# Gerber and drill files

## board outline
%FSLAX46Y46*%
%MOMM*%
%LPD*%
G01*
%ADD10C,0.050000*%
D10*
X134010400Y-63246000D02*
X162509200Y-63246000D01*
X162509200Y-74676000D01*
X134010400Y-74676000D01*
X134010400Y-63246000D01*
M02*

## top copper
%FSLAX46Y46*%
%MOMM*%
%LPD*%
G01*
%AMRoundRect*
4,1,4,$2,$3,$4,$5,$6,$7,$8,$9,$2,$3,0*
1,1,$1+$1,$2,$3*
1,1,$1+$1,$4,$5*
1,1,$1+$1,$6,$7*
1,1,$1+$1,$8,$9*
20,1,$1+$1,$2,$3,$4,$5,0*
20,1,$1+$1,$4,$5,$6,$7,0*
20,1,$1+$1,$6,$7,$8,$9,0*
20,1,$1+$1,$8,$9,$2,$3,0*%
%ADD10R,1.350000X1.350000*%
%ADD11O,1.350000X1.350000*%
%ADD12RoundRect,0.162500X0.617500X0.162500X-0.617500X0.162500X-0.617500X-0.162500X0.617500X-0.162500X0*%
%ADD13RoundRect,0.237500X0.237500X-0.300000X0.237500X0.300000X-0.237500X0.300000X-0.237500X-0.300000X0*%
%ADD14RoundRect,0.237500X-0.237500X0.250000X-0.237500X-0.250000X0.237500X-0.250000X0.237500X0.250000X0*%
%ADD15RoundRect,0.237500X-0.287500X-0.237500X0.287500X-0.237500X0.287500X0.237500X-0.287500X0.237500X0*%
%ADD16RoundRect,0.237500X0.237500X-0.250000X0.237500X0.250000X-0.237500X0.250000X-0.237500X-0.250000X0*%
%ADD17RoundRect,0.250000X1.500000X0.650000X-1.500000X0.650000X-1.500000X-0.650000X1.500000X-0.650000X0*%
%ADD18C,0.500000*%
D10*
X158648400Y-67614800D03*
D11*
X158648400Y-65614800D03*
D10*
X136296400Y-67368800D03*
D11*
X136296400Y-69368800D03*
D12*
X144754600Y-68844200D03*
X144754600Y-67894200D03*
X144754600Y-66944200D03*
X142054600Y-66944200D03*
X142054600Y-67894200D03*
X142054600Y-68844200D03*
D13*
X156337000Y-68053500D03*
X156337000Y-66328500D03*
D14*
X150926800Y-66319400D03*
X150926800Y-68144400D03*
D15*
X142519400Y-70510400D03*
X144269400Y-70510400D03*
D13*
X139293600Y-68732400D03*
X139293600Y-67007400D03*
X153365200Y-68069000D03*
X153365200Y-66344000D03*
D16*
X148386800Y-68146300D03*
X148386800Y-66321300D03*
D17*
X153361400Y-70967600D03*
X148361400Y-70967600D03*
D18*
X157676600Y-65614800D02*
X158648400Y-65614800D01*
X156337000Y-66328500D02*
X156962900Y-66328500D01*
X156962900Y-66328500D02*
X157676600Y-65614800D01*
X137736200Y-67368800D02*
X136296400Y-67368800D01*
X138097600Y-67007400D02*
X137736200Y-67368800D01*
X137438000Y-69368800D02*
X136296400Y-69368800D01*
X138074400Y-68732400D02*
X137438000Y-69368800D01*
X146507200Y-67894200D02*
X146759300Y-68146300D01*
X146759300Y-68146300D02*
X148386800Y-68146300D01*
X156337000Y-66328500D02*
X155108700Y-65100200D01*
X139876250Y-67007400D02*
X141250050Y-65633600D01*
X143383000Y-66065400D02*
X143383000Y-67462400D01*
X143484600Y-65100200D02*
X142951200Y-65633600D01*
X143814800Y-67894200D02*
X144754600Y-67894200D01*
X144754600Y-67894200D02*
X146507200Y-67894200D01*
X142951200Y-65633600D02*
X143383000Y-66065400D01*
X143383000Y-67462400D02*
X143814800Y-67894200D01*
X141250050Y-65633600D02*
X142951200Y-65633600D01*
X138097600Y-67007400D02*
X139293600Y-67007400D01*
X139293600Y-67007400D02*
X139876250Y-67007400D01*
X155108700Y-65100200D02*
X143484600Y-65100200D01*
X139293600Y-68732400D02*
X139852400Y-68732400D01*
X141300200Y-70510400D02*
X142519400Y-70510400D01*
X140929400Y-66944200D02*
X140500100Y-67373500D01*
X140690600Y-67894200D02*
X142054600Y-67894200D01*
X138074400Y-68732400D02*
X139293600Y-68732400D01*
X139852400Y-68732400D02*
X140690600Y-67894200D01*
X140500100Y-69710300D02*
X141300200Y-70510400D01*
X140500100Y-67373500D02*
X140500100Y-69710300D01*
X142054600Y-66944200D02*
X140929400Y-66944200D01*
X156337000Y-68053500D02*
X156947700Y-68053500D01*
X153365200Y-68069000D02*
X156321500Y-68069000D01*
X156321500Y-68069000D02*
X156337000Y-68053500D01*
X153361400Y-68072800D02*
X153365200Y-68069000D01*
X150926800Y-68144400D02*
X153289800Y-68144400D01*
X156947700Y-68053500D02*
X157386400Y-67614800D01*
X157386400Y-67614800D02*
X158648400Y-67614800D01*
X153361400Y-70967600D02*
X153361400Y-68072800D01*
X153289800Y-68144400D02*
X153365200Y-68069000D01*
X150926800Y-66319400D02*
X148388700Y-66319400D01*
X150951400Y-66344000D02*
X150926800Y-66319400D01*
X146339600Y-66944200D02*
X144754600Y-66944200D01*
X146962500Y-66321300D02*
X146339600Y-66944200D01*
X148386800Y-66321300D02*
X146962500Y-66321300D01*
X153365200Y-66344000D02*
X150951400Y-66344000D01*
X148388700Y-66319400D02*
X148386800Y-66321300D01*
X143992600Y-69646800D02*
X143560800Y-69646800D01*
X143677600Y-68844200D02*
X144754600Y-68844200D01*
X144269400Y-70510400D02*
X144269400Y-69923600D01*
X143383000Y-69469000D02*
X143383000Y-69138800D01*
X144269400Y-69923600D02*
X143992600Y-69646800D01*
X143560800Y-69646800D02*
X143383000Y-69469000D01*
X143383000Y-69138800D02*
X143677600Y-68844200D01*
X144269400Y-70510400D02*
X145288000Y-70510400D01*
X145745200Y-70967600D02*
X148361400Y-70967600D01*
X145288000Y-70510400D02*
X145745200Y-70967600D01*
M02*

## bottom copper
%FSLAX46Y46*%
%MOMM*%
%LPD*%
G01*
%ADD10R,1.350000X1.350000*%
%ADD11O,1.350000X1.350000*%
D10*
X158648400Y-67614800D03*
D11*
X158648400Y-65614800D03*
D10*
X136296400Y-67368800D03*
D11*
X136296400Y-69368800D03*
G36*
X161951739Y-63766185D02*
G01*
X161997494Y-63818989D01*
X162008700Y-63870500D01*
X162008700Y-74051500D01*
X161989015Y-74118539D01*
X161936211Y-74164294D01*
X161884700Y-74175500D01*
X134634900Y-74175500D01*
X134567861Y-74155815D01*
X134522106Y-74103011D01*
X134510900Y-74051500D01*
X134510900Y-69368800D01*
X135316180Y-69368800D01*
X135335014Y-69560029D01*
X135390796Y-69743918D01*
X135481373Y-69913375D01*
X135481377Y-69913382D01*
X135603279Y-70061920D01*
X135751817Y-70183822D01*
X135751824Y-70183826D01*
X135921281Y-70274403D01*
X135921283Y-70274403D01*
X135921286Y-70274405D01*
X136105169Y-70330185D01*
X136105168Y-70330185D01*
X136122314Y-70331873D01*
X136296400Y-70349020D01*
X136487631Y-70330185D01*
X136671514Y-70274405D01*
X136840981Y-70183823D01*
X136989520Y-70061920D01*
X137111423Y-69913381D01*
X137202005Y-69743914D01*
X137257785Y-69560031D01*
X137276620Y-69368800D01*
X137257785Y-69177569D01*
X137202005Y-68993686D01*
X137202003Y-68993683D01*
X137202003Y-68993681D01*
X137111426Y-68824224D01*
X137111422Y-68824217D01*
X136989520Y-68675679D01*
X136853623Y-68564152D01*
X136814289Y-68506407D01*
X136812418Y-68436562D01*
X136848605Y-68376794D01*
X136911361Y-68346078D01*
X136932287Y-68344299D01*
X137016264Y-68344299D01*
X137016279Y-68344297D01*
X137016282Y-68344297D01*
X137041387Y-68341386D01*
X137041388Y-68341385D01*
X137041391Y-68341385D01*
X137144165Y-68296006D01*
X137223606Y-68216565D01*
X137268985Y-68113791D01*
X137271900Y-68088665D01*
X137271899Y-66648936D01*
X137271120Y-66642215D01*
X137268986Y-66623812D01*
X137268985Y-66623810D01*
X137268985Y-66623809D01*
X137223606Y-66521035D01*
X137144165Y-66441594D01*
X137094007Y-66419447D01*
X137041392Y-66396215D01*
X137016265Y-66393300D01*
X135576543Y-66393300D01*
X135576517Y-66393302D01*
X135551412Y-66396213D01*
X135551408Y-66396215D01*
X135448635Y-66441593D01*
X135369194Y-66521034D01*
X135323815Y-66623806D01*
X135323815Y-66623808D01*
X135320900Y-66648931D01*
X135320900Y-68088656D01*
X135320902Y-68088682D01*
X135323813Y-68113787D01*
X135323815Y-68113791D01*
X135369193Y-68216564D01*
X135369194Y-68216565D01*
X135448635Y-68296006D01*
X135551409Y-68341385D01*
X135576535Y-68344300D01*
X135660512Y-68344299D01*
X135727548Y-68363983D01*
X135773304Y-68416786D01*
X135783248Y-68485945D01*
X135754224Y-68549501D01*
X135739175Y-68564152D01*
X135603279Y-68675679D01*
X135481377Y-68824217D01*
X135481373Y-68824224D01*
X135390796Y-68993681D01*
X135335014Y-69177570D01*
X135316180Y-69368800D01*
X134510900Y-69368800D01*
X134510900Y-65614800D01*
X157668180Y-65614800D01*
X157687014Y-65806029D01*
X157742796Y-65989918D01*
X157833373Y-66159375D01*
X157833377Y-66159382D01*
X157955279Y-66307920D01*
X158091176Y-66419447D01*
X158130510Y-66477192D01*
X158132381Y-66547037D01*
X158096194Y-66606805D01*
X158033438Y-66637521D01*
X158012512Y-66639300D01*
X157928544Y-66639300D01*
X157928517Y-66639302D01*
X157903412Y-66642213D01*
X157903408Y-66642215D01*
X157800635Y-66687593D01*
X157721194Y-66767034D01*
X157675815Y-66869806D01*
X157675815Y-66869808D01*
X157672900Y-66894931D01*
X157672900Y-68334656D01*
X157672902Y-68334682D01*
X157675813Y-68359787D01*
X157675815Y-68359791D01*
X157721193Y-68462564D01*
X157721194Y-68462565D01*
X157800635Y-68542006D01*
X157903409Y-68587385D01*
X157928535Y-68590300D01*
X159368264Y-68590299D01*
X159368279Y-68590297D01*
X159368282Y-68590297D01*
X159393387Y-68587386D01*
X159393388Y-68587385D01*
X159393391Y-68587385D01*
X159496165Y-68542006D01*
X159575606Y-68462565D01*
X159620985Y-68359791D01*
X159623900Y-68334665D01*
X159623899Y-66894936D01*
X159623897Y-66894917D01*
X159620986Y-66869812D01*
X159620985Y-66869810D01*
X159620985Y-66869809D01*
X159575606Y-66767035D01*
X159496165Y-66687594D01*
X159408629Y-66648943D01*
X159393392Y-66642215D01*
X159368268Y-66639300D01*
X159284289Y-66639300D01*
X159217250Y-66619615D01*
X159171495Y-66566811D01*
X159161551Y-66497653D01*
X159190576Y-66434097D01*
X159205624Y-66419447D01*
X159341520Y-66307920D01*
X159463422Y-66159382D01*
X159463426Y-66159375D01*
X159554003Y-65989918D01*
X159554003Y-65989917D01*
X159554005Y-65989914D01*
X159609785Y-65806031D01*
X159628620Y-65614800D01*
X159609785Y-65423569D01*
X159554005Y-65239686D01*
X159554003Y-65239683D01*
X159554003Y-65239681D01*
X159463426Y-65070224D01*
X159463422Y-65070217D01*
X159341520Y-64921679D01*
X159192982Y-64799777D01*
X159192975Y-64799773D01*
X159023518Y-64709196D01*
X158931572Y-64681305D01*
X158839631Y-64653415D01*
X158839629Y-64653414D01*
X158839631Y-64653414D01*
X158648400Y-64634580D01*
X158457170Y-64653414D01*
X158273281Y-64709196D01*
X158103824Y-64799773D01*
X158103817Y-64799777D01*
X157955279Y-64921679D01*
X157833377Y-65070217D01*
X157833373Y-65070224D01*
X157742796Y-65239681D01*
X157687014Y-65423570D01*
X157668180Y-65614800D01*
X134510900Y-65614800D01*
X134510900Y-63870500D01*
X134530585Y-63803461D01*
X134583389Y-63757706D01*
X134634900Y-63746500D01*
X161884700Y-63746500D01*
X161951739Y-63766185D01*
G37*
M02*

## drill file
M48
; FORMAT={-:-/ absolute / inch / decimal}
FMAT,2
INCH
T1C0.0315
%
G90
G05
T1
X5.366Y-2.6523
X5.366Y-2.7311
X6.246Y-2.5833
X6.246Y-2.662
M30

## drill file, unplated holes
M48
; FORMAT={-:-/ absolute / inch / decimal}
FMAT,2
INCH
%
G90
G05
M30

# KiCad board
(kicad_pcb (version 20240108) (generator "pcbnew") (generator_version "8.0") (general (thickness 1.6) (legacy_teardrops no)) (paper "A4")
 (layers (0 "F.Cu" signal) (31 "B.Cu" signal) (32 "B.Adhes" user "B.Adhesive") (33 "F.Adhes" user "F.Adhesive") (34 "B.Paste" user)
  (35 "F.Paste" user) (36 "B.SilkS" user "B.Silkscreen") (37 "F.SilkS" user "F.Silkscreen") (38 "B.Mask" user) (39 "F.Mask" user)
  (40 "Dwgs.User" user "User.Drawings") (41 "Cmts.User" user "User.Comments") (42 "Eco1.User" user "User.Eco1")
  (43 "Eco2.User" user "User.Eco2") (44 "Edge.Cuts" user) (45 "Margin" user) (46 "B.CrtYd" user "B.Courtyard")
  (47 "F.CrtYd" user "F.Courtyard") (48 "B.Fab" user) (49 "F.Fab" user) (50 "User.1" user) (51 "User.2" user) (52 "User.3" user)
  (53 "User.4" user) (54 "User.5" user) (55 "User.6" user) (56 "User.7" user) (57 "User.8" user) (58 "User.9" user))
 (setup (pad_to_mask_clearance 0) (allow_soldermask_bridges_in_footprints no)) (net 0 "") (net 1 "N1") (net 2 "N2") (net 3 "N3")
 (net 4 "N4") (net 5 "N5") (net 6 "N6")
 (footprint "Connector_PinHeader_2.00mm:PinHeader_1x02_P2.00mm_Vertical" (layer "F.Cu") (at 136.2964 67.3688)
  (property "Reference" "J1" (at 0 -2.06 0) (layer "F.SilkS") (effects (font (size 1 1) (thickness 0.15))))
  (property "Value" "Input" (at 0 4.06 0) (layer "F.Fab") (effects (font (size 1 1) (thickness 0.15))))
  (pad "1" thru_hole rect (at 0 0) (size 1.35 1.35) (drill 0.8) (layers "*.Cu" "*.Mask") (remove_unused_layers no) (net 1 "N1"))
  (pad "2" thru_hole oval (at 0 2) (size 1.35 1.35) (drill 0.8) (layers "*.Cu" "*.Mask") (remove_unused_layers no) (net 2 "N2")))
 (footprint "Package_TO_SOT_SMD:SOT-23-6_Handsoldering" (layer "F.Cu") (at 143.4046 67.8942 180)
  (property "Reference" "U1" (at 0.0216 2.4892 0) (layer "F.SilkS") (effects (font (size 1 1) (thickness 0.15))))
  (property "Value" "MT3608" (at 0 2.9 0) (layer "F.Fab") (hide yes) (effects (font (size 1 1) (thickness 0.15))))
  (pad "1" smd roundrect (at -1.35 -0.95 180) (size 1.56 0.65) (layers "F.Cu" "F.Paste" "F.Mask") (roundrect_rratio 0.25) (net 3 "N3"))
  (pad "2" smd roundrect (at -1.35 0 180) (size 1.56 0.65) (layers "F.Cu" "F.Paste" "F.Mask") (roundrect_rratio 0.25) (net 1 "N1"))
  (pad "3" smd roundrect (at -1.35 0.95 180) (size 1.56 0.65) (layers "F.Cu" "F.Paste" "F.Mask") (roundrect_rratio 0.25) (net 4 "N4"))
  (pad "4" smd roundrect (at 1.35 0.95 180) (size 1.56 0.65) (layers "F.Cu" "F.Paste" "F.Mask") (roundrect_rratio 0.25) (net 2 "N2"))
  (pad "5" smd roundrect (at 1.35 0 180) (size 1.56 0.65) (layers "F.Cu" "F.Paste" "F.Mask") (roundrect_rratio 0.25) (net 2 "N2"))
  (pad "6" smd roundrect (at 1.35 -0.95 180) (size 1.56 0.65) (layers "F.Cu" "F.Paste" "F.Mask") (roundrect_rratio 0.25) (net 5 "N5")))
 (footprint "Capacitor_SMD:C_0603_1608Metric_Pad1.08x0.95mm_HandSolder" (layer "F.Cu") (at 156.337 67.191 90)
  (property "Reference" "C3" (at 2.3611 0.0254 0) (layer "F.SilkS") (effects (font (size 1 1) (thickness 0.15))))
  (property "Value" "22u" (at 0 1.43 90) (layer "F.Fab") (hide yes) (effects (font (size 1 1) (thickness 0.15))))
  (pad "1" smd roundrect (at -0.8625 0 90) (size 1.075 0.95) (layers "F.Cu" "F.Paste" "F.Mask") (roundrect_rratio 0.25) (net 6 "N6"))
  (pad "2" smd roundrect (at 0.8625 0 90) (size 1.075 0.95) (layers "F.Cu" "F.Paste" "F.Mask") (roundrect_rratio 0.25) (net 1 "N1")))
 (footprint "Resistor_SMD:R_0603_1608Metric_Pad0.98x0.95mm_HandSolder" (layer "F.Cu") (at 150.9268 67.2319 -90)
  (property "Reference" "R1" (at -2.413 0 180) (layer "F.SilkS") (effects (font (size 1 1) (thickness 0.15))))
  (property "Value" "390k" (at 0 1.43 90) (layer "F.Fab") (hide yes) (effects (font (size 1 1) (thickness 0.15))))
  (pad "1" smd roundrect (at -0.9125 0 270) (size 0.975 0.95) (layers "F.Cu" "F.Paste" "F.Mask") (roundrect_rratio 0.25) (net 4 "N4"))
  (pad "2" smd roundrect (at 0.9125 0 270) (size 0.975 0.95) (layers "F.Cu" "F.Paste" "F.Mask") (roundrect_rratio 0.25) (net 6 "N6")))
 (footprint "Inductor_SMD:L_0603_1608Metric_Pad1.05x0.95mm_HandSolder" (layer "F.Cu") (at 143.3944 70.5104)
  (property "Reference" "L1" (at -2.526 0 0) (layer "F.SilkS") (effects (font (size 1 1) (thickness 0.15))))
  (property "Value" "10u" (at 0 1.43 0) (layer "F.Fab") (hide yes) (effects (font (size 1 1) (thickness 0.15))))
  (pad "1" smd roundrect (at -0.875 0) (size 1.05 0.95) (layers "F.Cu" "F.Paste" "F.Mask") (roundrect_rratio 0.25) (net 2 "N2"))
  (pad "2" smd roundrect (at 0.875 0) (size 1.05 0.95) (layers "F.Cu" "F.Paste" "F.Mask") (roundrect_rratio 0.25) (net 3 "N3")))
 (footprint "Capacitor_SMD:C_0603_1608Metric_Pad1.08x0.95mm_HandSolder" (layer "F.Cu") (at 139.2936 67.8699 90)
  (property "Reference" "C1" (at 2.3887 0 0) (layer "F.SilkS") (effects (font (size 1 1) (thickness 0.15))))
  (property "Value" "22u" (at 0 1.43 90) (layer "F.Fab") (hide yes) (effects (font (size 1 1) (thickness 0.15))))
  (pad "1" smd roundrect (at -0.8625 0 90) (size 1.075 0.95) (layers "F.Cu" "F.Paste" "F.Mask") (roundrect_rratio 0.25) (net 2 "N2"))
  (pad "2" smd roundrect (at 0.8625 0 90) (size 1.075 0.95) (layers "F.Cu" "F.Paste" "F.Mask") (roundrect_rratio 0.25) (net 1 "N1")))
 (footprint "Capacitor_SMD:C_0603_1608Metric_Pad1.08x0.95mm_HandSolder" (layer "F.Cu") (at 153.3652 67.2065 90)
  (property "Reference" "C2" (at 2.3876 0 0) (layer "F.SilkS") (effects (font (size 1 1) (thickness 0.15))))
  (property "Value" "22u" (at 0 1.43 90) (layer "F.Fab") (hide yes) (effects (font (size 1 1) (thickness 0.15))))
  (pad "1" smd roundrect (at -0.8625 0 90) (size 1.075 0.95) (layers "F.Cu" "F.Paste" "F.Mask") (roundrect_rratio 0.25) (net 6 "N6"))
  (pad "2" smd roundrect (at 0.8625 0 90) (size 1.075 0.95) (layers "F.Cu" "F.Paste" "F.Mask") (roundrect_rratio 0.25) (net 4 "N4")))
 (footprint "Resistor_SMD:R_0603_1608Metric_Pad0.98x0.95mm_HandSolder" (layer "F.Cu") (at 148.3868 67.2338 90)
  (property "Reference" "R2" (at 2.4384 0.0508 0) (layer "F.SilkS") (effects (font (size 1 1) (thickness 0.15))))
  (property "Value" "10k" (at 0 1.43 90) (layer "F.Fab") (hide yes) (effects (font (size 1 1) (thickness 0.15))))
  (pad "1" smd roundrect (at -0.9125 0 90) (size 0.975 0.95) (layers "F.Cu" "F.Paste" "F.Mask") (roundrect_rratio 0.25) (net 1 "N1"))
  (pad "2" smd roundrect (at 0.9125 0 90) (size 0.975 0.95) (layers "F.Cu" "F.Paste" "F.Mask") (roundrect_rratio 0.25) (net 4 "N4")))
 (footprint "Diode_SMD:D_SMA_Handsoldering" (layer "F.Cu") (at 150.8614 70.9676 180)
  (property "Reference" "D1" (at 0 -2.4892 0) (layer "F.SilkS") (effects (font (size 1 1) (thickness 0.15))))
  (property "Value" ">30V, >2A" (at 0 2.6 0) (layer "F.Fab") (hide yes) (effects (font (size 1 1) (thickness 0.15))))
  (pad "1" smd roundrect (at -2.5 0 180) (size 3.5 1.8) (layers "F.Cu" "F.Paste" "F.Mask") (roundrect_rratio 0.1388888889) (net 6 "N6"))
  (pad "2" smd roundrect (at 2.5 0 180) (size 3.5 1.8) (layers "F.Cu" "F.Paste" "F.Mask") (roundrect_rratio 0.1388888889) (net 3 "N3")))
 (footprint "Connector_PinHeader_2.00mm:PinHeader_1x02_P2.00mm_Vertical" (layer "F.Cu") (at 158.6484 67.6148 180)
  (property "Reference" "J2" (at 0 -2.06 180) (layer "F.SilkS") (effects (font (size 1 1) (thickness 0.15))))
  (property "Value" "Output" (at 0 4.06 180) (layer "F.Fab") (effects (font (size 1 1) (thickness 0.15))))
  (pad "1" thru_hole rect (at 0 0 180) (size 1.35 1.35) (drill 0.8) (layers "*.Cu" "*.Mask") (remove_unused_layers no) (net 6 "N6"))
  (pad "2" thru_hole oval (at 0 2 180) (size 1.35 1.35) (drill 0.8) (layers "*.Cu" "*.Mask") (remove_unused_layers no) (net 1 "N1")))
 (gr_rect (start 134.0104 63.246) (end 162.5092 74.676) (stroke (width 0.05) (type default)) (fill none) (layer "Edge.Cuts"))
 (segment (start 146.5072 67.8942) (end 146.7593 68.1463) (width 0.5) (layer "F.Cu") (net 1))
 (segment (start 146.7593 68.1463) (end 148.3868 68.1463) (width 0.5) (layer "F.Cu") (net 1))
 (segment (start 156.337 66.3285) (end 155.1087 65.1002) (width 0.5) (layer "F.Cu") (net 1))
 (segment (start 138.0976 67.0074) (end 137.7362 67.3688) (width 0.5) (layer "F.Cu") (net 1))
 (segment (start 139.87625 67.0074) (end 141.25005 65.6336) (width 0.5) (layer "F.Cu") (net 1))
 (segment (start 143.383 66.0654) (end 143.383 67.4624) (width 0.5) (layer "F.Cu") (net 1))
 (segment (start 143.4846 65.1002) (end 142.9512 65.6336) (width 0.5) (layer "F.Cu") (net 1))
 (segment (start 156.9629 66.3285) (end 157.6766 65.6148) (width 0.5) (layer "F.Cu") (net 1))
 (segment (start 143.8148 67.8942) (end 144.7546 67.8942) (width 0.5) (layer "F.Cu") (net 1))
 (segment (start 144.7546 67.8942) (end 146.5072 67.8942) (width 0.5) (layer "F.Cu") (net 1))
 (segment (start 156.337 66.3285) (end 156.9629 66.3285) (width 0.5) (layer "F.Cu") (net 1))
 (segment (start 142.9512 65.6336) (end 143.383 66.0654) (width 0.5) (layer "F.Cu") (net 1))
 (segment (start 143.383 67.4624) (end 143.8148 67.8942) (width 0.5) (layer "F.Cu") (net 1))
 (segment (start 141.25005 65.6336) (end 142.9512 65.6336) (width 0.5) (layer "F.Cu") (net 1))
 (segment (start 138.0976 67.0074) (end 139.2936 67.0074) (width 0.5) (layer "F.Cu") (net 1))
 (segment (start 137.7362 67.3688) (end 136.2964 67.3688) (width 0.5) (layer "F.Cu") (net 1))
 (segment (start 157.6766 65.6148) (end 158.6484 65.6148) (width 0.5) (layer "F.Cu") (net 1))
 (segment (start 139.2936 67.0074) (end 139.87625 67.0074) (width 0.5) (layer "F.Cu") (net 1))
 (segment (start 155.1087 65.1002) (end 143.4846 65.1002) (width 0.5) (layer "F.Cu") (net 1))
 (segment (start 137.438 69.3688) (end 136.2964 69.3688) (width 0.5) (layer "F.Cu") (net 2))
 (segment (start 139.2936 68.7324) (end 139.8524 68.7324) (width 0.5) (layer "F.Cu") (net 2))
 (segment (start 141.3002 70.5104) (end 142.5194 70.5104) (width 0.5) (layer "F.Cu") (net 2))
 (segment (start 140.9294 66.9442) (end 140.5001 67.3735) (width 0.5) (layer "F.Cu") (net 2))
 (segment (start 140.6906 67.8942) (end 142.0546 67.8942) (width 0.5) (layer "F.Cu") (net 2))
 (segment (start 138.0744 68.7324) (end 139.2936 68.7324) (width 0.5) (layer "F.Cu") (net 2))
 (segment (start 139.8524 68.7324) (end 140.6906 67.8942) (width 0.5) (layer "F.Cu") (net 2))
 (segment (start 140.5001 69.7103) (end 141.3002 70.5104) (width 0.5) (layer "F.Cu") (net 2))
 (segment (start 138.0744 68.7324) (end 137.438 69.3688) (width 0.5) (layer "F.Cu") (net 2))
 (segment (start 140.5001 67.3735) (end 140.5001 69.7103) (width 0.5) (layer "F.Cu") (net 2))
 (segment (start 142.0546 66.9442) (end 140.9294 66.9442) (width 0.5) (layer "F.Cu") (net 2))
 (segment (start 156.337 68.0535) (end 156.9477 68.0535) (width 0.5) (layer "F.Cu") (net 6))
 (segment (start 153.3652 68.069) (end 156.3215 68.069) (width 0.5) (layer "F.Cu") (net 6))
 (segment (start 156.3215 68.069) (end 156.337 68.0535) (width 0.5) (layer "F.Cu") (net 6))
 (segment (start 153.3614 68.0728) (end 153.3652 68.069) (width 0.5) (layer "F.Cu") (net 6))
 (segment (start 150.9268 68.1444) (end 153.2898 68.1444) (width 0.5) (layer "F.Cu") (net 6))
 (segment (start 156.9477 68.0535) (end 157.3864 67.6148) (width 0.5) (layer "F.Cu") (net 6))
 (segment (start 157.3864 67.6148) (end 158.6484 67.6148) (width 0.5) (layer "F.Cu") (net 6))
 (segment (start 153.3614 70.9676) (end 153.3614 68.0728) (width 0.5) (layer "F.Cu") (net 6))
 (segment (start 153.2898 68.1444) (end 153.3652 68.069) (width 0.5) (layer "F.Cu") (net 6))
 (segment (start 150.9268 66.3194) (end 148.3887 66.3194) (width 0.5) (layer "F.Cu") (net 4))
 (segment (start 150.9514 66.344) (end 150.9268 66.3194) (width 0.5) (layer "F.Cu") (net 4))
 (segment (start 146.3396 66.9442) (end 144.7546 66.9442) (width 0.5) (layer "F.Cu") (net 4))
 (segment (start 146.9625 66.3213) (end 146.3396 66.9442) (width 0.5) (layer "F.Cu") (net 4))
 (segment (start 148.3868 66.3213) (end 146.9625 66.3213) (width 0.5) (layer "F.Cu") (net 4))
 (segment (start 153.3652 66.344) (end 150.9514 66.344) (width 0.5) (layer "F.Cu") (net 4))
 (segment (start 148.3887 66.3194) (end 148.3868 66.3213) (width 0.5) (layer "F.Cu") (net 4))
 (segment (start 143.9926 69.6468) (end 143.5608 69.6468) (width 0.5) (layer "F.Cu") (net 3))
 (segment (start 143.6776 68.8442) (end 144.7546 68.8442) (width 0.5) (layer "F.Cu") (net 3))
 (segment (start 144.2694 70.5104) (end 144.2694 69.9236) (width 0.5) (layer "F.Cu") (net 3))
 (segment (start 143.383 69.469) (end 143.383 69.1388) (width 0.5) (layer "F.Cu") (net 3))
 (segment (start 144.2694 69.9236) (end 143.9926 69.6468) (width 0.5) (layer "F.Cu") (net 3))
 (segment (start 143.5608 69.6468) (end 143.383 69.469) (width 0.5) (layer "F.Cu") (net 3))
 (segment (start 143.383 69.1388) (end 143.6776 68.8442) (width 0.5) (layer "F.Cu") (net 3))
 (segment (start 144.2694 70.5104) (end 145.288 70.5104) (width 0.5) (layer "F.Cu") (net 3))
 (segment (start 145.7452 70.9676) (end 148.3614 70.9676) (width 0.5) (layer "F.Cu") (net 3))
 (segment (start 145.288 70.5104) (end 145.7452 70.9676) (width 0.5) (layer "F.Cu") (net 3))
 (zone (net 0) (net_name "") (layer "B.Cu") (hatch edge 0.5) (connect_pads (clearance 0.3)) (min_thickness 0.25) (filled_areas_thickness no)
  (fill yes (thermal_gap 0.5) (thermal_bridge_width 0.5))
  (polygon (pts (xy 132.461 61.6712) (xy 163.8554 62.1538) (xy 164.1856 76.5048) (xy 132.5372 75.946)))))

